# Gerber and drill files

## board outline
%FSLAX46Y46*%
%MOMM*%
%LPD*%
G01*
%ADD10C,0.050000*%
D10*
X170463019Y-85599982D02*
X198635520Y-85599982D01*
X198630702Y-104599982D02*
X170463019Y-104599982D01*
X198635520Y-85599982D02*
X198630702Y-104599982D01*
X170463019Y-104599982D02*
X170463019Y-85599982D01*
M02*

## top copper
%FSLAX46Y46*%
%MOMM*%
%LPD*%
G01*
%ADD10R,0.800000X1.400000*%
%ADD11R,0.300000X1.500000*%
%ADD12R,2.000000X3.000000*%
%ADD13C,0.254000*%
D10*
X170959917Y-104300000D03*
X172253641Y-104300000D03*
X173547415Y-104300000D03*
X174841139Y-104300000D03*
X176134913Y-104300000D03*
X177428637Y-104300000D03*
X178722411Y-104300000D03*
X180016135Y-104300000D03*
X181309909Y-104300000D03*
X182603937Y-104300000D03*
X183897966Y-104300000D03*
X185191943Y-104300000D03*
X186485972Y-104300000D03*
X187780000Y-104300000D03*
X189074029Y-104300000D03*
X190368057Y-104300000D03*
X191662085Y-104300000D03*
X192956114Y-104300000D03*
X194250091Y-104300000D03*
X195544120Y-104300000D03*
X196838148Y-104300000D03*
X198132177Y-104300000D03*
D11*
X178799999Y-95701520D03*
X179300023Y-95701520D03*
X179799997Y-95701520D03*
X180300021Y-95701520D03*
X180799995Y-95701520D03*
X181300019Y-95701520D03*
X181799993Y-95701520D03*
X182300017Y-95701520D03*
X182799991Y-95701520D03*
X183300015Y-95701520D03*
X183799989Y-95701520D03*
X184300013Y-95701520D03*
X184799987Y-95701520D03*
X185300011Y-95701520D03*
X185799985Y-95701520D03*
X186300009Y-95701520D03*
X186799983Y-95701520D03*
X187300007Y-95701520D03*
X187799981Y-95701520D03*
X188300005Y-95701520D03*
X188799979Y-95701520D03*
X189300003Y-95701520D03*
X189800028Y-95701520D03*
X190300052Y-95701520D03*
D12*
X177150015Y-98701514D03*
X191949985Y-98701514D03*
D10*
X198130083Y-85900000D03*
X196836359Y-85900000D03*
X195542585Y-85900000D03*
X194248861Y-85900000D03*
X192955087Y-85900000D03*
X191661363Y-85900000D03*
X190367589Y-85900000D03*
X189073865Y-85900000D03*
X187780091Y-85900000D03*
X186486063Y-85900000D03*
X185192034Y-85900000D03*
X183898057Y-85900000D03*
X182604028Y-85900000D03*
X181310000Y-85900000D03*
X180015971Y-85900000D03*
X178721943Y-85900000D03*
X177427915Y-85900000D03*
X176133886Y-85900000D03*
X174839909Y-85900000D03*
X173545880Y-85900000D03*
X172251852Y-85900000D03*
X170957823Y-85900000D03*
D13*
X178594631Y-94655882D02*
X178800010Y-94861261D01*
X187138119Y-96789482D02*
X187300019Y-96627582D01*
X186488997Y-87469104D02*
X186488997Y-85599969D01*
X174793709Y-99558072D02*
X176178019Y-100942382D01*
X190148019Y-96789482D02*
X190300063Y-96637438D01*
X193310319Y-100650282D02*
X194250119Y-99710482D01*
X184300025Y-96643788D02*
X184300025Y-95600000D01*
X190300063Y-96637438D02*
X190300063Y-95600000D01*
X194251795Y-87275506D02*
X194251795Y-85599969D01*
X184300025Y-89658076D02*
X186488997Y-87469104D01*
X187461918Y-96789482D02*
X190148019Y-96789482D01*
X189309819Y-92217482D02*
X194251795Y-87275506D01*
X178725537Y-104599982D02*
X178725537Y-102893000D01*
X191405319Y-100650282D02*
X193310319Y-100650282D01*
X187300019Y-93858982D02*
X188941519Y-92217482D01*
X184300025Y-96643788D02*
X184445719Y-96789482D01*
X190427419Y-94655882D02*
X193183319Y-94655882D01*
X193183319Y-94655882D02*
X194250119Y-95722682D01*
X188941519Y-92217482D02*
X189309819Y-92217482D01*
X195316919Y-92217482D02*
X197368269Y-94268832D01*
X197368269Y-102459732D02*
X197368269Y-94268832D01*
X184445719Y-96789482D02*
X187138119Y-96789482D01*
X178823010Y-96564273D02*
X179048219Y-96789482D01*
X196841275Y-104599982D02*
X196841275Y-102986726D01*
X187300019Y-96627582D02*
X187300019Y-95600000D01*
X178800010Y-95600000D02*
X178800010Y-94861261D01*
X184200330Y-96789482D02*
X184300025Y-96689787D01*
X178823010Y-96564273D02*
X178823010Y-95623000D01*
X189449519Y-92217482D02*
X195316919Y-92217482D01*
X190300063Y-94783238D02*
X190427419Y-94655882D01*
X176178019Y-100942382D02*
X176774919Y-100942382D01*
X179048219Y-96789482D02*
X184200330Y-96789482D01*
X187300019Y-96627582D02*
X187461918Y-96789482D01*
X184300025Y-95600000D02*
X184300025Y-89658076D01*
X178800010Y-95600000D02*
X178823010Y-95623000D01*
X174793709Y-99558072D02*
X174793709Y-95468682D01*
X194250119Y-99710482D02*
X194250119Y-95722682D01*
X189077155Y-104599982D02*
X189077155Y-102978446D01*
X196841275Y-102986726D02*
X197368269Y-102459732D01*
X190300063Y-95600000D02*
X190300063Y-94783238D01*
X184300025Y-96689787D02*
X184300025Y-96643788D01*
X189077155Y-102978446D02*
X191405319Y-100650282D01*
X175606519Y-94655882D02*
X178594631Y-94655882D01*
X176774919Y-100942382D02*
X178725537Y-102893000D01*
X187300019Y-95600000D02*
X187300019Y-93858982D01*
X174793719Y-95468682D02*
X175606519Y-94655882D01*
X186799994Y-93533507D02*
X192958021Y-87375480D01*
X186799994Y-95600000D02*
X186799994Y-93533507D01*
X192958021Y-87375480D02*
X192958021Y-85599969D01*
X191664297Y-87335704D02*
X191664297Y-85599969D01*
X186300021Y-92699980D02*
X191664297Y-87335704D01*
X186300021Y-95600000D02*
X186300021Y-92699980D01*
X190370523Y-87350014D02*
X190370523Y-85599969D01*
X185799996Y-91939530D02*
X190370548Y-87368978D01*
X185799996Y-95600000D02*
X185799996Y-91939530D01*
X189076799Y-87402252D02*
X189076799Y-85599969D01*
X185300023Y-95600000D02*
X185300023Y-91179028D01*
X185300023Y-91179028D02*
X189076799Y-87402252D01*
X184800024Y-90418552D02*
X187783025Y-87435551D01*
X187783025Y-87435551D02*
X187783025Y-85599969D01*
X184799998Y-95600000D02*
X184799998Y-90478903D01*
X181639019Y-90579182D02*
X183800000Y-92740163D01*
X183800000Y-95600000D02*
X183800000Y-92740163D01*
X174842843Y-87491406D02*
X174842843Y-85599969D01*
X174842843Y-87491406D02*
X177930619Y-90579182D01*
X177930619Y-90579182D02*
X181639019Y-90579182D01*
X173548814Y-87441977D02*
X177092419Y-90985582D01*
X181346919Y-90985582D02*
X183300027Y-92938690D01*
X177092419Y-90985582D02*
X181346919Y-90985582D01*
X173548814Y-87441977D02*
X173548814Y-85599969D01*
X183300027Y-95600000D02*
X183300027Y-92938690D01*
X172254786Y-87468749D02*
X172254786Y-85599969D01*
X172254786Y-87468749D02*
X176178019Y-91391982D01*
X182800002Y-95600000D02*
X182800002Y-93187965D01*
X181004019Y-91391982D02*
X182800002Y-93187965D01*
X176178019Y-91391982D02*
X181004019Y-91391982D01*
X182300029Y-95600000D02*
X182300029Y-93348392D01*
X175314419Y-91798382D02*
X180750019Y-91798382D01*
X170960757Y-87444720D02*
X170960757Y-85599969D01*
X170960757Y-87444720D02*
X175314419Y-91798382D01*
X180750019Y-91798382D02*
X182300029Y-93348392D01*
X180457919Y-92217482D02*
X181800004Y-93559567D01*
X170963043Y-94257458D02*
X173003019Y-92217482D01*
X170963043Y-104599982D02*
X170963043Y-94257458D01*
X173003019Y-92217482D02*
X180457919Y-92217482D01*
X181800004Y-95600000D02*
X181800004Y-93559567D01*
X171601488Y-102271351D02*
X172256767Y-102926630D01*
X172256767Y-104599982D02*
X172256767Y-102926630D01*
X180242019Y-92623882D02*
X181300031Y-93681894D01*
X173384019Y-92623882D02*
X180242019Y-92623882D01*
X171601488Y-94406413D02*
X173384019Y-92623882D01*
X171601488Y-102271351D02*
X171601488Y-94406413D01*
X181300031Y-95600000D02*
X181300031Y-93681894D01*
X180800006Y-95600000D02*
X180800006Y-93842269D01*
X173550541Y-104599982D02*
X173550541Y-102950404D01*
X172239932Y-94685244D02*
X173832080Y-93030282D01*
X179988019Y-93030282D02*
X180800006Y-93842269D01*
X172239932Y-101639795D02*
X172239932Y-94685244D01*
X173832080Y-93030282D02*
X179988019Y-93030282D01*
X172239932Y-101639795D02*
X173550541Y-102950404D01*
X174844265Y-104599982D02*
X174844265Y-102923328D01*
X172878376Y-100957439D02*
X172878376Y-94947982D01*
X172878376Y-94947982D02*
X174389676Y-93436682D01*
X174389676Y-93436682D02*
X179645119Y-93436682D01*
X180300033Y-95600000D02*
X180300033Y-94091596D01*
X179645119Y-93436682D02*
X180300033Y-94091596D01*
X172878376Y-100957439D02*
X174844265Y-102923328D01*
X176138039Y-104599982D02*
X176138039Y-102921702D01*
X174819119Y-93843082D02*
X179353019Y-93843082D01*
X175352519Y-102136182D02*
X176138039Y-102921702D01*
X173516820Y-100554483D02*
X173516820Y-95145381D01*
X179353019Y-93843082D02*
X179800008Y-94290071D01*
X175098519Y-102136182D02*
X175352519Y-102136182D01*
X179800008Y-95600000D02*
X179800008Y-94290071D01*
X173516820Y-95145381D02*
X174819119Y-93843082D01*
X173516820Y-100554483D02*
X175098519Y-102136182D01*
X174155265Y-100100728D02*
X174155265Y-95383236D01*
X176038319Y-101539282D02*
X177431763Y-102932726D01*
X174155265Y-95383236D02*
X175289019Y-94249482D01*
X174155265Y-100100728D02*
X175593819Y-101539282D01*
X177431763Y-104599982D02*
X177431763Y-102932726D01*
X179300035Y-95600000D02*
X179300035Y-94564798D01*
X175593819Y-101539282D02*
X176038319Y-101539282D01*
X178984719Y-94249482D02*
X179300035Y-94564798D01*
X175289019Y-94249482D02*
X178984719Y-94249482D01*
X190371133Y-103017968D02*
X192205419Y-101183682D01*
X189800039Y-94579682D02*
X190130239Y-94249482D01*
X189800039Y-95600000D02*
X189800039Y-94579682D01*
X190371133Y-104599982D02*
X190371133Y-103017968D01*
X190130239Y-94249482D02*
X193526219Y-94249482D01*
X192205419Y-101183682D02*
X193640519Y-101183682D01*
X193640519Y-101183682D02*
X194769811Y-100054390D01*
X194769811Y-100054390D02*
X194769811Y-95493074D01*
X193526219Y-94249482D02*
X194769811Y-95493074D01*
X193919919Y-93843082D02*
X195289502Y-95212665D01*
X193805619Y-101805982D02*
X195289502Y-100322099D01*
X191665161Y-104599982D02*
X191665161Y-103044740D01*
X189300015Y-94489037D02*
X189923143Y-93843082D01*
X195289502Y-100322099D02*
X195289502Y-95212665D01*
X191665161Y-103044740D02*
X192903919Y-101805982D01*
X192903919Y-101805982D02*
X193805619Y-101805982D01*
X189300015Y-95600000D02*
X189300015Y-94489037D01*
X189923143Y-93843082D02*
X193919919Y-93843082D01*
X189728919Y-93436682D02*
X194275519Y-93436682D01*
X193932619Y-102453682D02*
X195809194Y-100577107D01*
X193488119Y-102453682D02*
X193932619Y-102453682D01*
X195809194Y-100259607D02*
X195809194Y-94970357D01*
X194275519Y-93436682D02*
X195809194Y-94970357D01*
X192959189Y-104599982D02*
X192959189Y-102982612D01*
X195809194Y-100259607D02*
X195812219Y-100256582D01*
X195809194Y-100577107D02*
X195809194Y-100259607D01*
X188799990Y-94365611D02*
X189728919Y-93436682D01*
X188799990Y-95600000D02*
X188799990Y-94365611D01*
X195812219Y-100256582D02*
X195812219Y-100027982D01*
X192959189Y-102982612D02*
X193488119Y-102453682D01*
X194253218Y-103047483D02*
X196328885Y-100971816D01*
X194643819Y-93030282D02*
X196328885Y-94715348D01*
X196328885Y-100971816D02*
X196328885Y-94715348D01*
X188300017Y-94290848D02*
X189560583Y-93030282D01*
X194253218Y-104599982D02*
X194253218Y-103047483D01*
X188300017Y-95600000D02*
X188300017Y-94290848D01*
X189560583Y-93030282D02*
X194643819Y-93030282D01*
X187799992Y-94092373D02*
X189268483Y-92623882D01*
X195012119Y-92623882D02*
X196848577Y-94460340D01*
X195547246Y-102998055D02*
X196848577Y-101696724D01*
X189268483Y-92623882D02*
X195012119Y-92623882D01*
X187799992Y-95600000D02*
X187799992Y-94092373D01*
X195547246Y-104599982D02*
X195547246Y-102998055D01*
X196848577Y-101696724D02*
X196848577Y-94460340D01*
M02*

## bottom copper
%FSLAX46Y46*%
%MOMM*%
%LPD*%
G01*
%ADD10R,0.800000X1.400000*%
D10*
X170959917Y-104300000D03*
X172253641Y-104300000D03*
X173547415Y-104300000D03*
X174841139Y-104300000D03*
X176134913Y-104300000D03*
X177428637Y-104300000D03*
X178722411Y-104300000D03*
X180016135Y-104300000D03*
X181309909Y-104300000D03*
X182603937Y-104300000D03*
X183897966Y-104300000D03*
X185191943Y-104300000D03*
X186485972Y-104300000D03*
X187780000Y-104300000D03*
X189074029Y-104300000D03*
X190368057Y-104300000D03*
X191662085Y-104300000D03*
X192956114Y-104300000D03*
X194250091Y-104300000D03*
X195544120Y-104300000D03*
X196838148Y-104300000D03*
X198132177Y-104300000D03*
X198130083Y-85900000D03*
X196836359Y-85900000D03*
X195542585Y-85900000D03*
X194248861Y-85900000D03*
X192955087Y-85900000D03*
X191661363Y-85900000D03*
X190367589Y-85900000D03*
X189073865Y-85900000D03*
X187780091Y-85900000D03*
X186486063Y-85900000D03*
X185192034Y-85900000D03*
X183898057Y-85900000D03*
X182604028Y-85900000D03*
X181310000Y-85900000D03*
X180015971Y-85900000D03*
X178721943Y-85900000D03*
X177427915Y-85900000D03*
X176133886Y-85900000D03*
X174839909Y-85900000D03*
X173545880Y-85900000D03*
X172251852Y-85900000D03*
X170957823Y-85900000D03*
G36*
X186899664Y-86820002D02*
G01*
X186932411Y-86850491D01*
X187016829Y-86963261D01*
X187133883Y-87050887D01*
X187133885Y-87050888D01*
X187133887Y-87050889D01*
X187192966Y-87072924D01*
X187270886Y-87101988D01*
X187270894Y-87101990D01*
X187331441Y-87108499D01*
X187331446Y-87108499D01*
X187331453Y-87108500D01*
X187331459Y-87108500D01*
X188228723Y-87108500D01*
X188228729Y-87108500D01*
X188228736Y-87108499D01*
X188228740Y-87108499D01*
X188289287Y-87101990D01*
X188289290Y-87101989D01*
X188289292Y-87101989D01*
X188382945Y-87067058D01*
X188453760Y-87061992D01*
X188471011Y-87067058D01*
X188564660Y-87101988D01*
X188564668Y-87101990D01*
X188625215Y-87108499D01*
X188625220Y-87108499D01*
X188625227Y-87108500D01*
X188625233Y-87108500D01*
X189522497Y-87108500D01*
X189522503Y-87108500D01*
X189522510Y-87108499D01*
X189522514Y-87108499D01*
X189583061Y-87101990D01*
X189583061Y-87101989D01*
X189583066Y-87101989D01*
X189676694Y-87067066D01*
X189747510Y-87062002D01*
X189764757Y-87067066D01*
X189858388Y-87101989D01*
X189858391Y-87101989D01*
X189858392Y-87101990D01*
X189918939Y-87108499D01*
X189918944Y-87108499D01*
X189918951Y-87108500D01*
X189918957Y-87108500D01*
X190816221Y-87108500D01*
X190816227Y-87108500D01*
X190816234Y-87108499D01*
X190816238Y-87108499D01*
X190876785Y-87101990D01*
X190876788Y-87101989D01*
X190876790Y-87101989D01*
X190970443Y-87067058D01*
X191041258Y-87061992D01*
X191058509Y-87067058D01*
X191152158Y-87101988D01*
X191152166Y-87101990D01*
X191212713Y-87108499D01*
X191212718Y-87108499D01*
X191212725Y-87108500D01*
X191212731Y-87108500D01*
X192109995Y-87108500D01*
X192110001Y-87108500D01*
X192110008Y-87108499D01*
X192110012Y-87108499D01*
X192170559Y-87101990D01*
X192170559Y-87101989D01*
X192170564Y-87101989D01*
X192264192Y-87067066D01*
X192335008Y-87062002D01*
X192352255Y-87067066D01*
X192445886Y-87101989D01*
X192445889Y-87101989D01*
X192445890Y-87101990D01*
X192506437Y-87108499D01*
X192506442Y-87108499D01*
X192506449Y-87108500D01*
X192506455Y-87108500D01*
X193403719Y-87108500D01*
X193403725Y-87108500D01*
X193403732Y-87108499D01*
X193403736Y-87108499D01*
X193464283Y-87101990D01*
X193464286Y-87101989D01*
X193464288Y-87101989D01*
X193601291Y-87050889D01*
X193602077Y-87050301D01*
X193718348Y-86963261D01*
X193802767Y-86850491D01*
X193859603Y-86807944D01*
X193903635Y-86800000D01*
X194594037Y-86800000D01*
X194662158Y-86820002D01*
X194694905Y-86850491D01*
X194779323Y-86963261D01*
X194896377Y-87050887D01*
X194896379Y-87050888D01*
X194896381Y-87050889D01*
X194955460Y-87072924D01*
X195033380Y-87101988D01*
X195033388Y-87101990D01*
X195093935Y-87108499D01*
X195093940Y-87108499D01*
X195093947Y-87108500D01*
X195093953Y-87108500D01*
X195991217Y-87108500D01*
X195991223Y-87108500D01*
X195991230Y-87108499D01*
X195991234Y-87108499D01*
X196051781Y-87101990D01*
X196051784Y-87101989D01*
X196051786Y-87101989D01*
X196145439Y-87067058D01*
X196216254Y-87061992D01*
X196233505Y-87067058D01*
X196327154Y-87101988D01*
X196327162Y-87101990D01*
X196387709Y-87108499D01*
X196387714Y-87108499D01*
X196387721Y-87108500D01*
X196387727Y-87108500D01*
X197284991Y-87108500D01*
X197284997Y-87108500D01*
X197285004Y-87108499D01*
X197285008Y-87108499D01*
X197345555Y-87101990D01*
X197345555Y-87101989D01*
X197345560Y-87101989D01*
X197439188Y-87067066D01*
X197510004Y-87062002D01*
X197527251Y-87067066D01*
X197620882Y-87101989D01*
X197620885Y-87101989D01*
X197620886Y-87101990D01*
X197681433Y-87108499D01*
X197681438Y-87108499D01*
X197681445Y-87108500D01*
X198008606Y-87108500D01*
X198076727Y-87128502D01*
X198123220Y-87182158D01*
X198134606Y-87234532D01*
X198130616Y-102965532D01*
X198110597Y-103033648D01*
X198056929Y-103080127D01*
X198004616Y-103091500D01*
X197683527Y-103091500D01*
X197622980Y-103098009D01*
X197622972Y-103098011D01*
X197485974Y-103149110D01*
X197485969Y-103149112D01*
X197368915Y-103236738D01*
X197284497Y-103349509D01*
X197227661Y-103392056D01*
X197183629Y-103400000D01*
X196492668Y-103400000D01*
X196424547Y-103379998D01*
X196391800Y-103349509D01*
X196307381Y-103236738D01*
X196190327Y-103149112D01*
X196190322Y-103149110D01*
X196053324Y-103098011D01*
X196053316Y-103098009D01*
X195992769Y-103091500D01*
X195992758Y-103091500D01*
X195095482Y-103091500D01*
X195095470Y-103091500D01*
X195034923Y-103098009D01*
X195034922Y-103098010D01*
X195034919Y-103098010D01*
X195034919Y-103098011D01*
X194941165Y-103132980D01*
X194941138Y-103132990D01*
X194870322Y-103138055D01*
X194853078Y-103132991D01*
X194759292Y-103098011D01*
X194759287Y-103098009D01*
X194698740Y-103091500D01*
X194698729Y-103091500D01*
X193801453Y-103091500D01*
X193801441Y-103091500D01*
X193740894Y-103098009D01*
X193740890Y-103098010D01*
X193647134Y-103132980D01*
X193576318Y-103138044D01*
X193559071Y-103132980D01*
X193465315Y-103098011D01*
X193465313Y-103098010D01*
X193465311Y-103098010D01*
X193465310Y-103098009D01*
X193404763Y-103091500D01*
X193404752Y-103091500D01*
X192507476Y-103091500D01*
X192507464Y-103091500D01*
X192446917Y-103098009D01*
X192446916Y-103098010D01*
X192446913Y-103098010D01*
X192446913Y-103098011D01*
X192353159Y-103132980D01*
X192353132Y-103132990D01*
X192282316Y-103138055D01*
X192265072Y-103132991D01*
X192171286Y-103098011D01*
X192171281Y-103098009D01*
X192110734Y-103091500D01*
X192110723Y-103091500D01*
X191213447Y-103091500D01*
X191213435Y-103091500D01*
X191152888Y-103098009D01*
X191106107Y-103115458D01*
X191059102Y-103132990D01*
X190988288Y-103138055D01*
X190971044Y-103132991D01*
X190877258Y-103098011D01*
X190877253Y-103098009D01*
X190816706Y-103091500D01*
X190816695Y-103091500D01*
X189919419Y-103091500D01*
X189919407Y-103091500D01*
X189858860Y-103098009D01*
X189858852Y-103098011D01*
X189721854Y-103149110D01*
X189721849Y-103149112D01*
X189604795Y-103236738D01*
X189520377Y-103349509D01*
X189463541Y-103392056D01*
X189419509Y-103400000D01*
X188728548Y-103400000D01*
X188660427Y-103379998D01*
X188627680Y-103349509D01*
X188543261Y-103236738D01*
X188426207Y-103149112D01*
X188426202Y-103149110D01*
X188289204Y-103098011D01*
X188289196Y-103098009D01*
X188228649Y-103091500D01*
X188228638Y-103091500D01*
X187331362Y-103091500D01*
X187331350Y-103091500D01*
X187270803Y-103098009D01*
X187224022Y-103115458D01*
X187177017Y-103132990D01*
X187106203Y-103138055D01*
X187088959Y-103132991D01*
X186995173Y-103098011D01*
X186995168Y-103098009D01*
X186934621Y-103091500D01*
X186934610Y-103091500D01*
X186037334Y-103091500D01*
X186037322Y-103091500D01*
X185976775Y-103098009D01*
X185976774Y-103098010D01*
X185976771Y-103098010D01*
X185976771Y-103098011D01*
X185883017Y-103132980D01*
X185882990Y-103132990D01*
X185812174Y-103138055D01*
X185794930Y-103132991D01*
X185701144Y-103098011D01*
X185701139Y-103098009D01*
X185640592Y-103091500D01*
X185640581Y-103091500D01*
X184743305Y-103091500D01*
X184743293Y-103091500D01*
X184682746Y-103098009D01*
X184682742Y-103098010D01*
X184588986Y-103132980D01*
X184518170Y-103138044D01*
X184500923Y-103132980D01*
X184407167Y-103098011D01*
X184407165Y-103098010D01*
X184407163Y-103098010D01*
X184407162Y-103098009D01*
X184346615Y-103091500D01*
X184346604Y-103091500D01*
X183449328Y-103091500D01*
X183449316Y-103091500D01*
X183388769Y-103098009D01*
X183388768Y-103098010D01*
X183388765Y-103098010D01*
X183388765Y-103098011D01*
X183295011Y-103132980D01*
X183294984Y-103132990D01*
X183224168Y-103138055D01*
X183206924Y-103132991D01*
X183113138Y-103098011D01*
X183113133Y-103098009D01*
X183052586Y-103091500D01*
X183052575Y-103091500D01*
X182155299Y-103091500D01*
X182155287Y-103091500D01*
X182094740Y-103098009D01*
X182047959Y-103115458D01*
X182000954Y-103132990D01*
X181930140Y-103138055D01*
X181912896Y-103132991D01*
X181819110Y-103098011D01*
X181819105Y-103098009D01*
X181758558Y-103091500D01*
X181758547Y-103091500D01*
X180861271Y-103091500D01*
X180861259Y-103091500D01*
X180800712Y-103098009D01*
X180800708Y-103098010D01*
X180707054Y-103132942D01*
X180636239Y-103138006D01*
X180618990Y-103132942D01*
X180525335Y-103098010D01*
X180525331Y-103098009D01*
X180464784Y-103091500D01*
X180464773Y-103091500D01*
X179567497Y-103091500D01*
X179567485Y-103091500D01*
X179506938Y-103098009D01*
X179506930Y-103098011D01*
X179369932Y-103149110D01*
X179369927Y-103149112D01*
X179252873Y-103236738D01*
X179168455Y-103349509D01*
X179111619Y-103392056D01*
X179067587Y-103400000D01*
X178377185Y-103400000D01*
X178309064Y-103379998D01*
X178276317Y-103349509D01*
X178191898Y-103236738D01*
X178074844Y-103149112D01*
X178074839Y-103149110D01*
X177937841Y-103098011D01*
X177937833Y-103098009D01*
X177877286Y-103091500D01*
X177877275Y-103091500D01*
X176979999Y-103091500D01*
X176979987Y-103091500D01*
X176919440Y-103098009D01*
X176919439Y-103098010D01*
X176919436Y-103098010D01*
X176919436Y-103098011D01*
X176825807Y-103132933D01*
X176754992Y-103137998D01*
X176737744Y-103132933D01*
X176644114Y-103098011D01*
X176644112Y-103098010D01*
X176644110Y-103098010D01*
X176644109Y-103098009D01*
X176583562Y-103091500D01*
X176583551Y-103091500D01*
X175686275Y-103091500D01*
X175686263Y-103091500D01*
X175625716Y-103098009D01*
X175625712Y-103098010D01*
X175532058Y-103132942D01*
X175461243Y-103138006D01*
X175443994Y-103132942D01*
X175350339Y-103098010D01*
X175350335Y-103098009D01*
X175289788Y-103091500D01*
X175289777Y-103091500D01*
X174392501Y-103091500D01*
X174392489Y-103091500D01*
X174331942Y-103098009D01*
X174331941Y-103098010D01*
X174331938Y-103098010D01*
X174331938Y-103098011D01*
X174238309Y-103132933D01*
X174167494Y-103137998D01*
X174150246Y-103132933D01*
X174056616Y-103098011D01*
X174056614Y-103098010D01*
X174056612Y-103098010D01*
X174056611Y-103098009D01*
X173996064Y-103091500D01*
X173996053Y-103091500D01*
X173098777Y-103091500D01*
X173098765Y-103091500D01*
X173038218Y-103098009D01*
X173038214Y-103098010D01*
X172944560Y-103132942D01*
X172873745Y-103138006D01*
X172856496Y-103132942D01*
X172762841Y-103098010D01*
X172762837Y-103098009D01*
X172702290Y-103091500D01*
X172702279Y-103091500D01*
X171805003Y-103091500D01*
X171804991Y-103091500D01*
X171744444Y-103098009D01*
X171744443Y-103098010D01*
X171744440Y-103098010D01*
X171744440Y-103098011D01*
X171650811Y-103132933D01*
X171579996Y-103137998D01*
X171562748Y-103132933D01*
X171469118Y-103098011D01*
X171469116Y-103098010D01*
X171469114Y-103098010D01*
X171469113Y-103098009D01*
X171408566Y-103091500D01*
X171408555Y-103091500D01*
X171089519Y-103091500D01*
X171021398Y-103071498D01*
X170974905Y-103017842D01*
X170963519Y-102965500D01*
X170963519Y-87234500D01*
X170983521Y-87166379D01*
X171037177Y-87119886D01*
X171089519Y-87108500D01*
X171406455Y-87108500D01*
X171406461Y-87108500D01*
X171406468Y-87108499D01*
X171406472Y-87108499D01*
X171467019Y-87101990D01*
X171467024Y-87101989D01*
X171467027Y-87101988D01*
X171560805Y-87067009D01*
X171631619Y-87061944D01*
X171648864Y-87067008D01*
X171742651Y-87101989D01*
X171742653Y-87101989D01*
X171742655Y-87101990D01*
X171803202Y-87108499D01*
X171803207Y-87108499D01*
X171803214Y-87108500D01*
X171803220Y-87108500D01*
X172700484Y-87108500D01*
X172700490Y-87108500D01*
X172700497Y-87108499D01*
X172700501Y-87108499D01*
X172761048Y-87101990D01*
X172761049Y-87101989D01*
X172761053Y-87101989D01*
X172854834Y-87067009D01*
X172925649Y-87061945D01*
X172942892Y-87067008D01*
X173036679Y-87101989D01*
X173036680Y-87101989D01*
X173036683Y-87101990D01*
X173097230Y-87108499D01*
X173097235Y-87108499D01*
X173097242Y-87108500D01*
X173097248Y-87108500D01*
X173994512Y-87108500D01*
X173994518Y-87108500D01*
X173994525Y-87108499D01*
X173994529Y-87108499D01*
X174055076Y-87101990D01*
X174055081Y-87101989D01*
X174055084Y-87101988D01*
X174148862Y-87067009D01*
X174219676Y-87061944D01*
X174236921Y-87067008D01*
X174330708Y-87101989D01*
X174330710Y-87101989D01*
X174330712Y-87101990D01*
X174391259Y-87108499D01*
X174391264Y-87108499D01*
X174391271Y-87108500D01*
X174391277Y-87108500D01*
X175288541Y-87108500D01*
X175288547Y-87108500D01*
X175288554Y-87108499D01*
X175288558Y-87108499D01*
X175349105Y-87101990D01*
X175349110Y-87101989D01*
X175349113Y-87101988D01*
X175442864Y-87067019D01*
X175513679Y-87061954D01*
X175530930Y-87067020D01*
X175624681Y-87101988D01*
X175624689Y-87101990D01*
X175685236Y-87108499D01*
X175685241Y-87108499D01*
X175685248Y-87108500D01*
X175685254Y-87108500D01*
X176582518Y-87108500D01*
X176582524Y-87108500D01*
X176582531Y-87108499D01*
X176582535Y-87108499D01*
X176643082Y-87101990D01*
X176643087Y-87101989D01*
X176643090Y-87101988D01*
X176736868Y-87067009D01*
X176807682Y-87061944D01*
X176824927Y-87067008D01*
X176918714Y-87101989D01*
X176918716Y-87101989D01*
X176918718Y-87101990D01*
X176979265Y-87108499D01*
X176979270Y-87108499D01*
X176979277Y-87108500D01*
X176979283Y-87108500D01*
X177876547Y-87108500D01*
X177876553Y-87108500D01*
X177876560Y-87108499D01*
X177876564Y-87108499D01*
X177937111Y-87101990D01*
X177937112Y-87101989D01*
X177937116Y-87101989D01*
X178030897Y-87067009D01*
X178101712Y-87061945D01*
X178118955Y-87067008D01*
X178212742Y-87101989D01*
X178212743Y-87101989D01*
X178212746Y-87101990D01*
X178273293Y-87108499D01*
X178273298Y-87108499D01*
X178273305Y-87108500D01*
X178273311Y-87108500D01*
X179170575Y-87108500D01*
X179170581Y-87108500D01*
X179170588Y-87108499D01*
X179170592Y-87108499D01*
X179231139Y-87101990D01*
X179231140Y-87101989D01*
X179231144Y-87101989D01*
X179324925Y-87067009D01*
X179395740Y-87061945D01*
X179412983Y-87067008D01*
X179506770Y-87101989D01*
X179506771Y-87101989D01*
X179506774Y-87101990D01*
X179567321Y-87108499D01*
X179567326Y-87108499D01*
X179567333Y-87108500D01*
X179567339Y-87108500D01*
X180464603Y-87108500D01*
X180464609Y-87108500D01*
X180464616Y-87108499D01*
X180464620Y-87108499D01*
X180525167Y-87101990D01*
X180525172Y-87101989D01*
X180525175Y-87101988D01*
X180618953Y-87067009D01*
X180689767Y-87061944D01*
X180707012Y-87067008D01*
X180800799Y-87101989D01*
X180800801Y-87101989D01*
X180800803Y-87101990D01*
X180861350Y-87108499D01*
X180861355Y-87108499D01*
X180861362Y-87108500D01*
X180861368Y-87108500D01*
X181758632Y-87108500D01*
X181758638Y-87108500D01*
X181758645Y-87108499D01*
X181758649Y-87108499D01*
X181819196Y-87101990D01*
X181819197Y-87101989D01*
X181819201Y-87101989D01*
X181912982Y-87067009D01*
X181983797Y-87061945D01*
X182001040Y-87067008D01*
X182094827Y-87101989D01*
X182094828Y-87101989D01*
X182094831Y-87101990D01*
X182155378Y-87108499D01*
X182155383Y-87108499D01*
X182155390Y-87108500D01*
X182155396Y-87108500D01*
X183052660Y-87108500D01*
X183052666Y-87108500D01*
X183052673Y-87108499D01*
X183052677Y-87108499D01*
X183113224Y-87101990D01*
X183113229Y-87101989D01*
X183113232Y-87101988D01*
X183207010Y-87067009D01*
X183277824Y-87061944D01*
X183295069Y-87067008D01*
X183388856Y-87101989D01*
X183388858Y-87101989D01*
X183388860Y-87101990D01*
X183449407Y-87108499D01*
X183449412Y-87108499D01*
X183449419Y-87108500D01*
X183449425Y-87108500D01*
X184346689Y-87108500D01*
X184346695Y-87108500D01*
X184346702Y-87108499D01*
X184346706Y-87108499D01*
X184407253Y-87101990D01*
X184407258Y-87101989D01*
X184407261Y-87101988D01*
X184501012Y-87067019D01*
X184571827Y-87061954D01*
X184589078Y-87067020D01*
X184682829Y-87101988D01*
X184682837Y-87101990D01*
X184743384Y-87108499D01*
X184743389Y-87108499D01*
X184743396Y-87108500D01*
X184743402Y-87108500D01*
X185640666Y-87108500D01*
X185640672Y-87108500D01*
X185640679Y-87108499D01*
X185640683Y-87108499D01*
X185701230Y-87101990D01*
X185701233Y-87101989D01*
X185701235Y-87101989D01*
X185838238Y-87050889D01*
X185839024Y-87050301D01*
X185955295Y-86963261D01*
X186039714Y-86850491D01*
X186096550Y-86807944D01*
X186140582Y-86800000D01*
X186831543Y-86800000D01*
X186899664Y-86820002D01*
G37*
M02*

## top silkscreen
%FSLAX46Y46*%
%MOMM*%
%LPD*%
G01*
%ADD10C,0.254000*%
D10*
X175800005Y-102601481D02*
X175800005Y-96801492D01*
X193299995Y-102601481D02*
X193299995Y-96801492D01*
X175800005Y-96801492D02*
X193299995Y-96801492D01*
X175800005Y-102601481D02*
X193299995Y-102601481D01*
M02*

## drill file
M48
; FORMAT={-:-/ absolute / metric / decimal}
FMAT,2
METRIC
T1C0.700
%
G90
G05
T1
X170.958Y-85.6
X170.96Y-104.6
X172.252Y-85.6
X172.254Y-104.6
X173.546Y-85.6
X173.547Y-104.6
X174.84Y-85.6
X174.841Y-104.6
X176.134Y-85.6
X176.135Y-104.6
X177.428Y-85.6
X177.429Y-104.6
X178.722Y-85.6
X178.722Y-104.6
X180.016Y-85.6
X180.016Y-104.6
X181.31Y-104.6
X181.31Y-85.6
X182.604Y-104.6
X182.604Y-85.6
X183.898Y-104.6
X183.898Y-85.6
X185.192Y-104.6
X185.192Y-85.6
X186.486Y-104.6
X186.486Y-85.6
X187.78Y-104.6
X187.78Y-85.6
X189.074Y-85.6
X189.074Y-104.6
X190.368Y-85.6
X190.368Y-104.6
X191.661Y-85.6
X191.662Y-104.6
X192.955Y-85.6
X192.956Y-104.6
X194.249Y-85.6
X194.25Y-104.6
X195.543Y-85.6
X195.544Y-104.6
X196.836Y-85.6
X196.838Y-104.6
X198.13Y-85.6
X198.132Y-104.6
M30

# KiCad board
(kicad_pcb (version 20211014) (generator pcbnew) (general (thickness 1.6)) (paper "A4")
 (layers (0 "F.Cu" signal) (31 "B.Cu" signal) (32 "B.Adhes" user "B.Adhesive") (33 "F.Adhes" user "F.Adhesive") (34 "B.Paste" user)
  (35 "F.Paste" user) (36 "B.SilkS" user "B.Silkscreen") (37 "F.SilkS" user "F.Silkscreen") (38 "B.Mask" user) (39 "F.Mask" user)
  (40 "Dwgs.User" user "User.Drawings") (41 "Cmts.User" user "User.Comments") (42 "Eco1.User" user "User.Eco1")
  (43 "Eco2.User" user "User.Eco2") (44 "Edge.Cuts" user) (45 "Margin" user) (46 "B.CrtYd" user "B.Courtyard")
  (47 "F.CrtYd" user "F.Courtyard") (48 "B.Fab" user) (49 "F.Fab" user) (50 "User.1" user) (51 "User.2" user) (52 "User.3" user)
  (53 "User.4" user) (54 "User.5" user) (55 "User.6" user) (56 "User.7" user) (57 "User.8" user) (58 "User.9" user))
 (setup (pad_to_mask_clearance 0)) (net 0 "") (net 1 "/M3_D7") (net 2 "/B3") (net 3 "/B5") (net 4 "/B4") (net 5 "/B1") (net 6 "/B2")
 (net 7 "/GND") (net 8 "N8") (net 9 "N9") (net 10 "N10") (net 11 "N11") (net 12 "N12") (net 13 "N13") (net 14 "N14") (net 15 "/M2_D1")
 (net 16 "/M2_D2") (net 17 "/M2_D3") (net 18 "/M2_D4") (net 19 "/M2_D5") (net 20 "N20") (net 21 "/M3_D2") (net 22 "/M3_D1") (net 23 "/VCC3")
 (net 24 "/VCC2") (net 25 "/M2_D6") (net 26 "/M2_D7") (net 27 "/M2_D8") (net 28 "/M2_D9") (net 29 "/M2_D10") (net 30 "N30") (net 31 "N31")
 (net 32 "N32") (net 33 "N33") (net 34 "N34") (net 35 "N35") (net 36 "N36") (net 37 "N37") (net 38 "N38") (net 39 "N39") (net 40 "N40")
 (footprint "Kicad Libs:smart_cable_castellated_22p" (layer "F.Cu") (at 184.58 104.4 180)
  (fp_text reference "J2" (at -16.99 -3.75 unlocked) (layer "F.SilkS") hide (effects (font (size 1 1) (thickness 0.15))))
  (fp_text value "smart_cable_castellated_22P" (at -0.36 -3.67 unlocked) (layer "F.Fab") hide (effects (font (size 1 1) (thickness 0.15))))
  (pad "1" thru_hole rect (at 13.620083 -0.2 180) (size 0.8 1.4) (drill 0.7 (offset 0 0.3)) (layers *.Cu *.Mask) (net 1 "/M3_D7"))
  (pad "2" thru_hole rect (at 12.326359 -0.2 180) (size 0.8 1.4) (drill 0.7 (offset 0 0.3)) (layers *.Cu *.Mask) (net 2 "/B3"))
  (pad "3" thru_hole rect (at 11.032585 -0.2 180) (size 0.8 1.4) (drill 0.7 (offset 0 0.3)) (layers *.Cu *.Mask) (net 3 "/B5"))
  (pad "4" thru_hole rect (at 9.738861 -0.2 180) (size 0.8 1.4) (drill 0.7 (offset 0 0.3)) (layers *.Cu *.Mask) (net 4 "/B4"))
  (pad "5" thru_hole rect (at 8.445087 -0.2 180) (size 0.8 1.4) (drill 0.7 (offset 0 0.3)) (layers *.Cu *.Mask) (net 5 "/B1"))
  (pad "6" thru_hole rect (at 7.151363 -0.2 180) (size 0.8 1.4) (drill 0.7 (offset 0 0.3)) (layers *.Cu *.Mask) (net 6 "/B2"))
  (pad "7" thru_hole rect (at 5.857589 -0.2 180) (size 0.8 1.4) (drill 0.7 (offset 0 0.3)) (layers *.Cu *.Mask) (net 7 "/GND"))
  (pad "8" thru_hole rect (at 4.563865 -0.2 180) (size 0.8 1.4) (drill 0.7 (offset 0 0.3)) (layers *.Cu *.Mask) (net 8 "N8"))
  (pad "9" thru_hole rect (at 3.270091 -0.2 180) (size 0.8 1.4) (drill 0.7 (offset 0 0.3)) (layers *.Cu *.Mask) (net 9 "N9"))
  (pad "10" thru_hole rect (at 1.976063 -0.2 180) (size 0.8 1.4) (drill 0.7 (offset 0 0.3)) (layers *.Cu *.Mask) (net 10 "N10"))
  (pad "11" thru_hole rect (at 0.682034 -0.2 180) (size 0.8 1.4) (drill 0.7 (offset 0 0.3)) (layers *.Cu *.Mask) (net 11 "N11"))
  (pad "12" thru_hole rect (at -0.611943 -0.2 180) (size 0.8 1.4) (drill 0.7 (offset 0 0.3)) (layers *.Cu *.Mask) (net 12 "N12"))
  (pad "13" thru_hole rect (at -1.905972 -0.2 180) (size 0.8 1.4) (drill 0.7 (offset 0 0.3)) (layers *.Cu *.Mask) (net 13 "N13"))
  (pad "14" thru_hole rect (at -3.2 -0.2 180) (size 0.8 1.4) (drill 0.7 (offset 0 0.3)) (layers *.Cu *.Mask) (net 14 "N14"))
  (pad "15" thru_hole rect (at -4.494029 -0.2 180) (size 0.8 1.4) (drill 0.7 (offset 0 0.3)) (layers *.Cu *.Mask) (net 7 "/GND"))
  (pad "16" thru_hole rect (at -5.788057 -0.2 180) (size 0.8 1.4) (drill 0.7 (offset 0 0.3)) (layers *.Cu *.Mask) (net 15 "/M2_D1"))
  (pad "17" thru_hole rect (at -7.082085 -0.2 180) (size 0.8 1.4) (drill 0.7 (offset 0 0.3)) (layers *.Cu *.Mask) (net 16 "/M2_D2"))
  (pad "18" thru_hole rect (at -8.376114 -0.2 180) (size 0.8 1.4) (drill 0.7 (offset 0 0.3)) (layers *.Cu *.Mask) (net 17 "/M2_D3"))
  (pad "19" thru_hole rect (at -9.670091 -0.2 180) (size 0.8 1.4) (drill 0.7 (offset 0 0.3)) (layers *.Cu *.Mask) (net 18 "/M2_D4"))
  (pad "20" thru_hole rect (at -10.96412 -0.2 180) (size 0.8 1.4) (drill 0.7 (offset 0 0.3)) (layers *.Cu *.Mask) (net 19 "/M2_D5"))
  (pad "21" thru_hole rect (at -12.258148 -0.2 180) (size 0.8 1.4) (drill 0.7 (offset 0 0.3)) (layers *.Cu *.Mask) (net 7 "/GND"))
  (pad "22" thru_hole rect (at -13.552177 -0.2 180) (size 0.8 1.4) (drill 0.7 (offset 0 0.3)) (layers *.Cu *.Mask) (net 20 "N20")))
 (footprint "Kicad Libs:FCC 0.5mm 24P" (layer "F.Cu") (at 184.55 100.14)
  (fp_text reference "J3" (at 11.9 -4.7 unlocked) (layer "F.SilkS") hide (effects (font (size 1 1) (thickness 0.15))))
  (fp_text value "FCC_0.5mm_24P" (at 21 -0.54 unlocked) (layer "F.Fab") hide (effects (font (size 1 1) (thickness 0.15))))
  (fp_line (start -8.749995 2.461481) (end -8.749995 -3.338508) (layer "F.SilkS") (width 0.254))
  (fp_line (start 8.749995 2.461481) (end 8.749995 -3.338508) (layer "F.SilkS") (width 0.254))
  (fp_line (start -8.749995 -3.338508) (end 8.749995 -3.338508) (layer "F.SilkS") (width 0.254))
  (fp_line (start -8.749995 2.461481) (end 8.749995 2.461481) (layer "F.SilkS") (width 0.254))
  (pad "1" smd rect (at -5.750001 -4.43848) (size 0.3 1.5) (layers "F.Cu" "F.Paste" "F.Mask") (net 7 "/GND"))
  (pad "2" smd rect (at -5.249977 -4.43848) (size 0.3 1.5) (layers "F.Cu" "F.Paste" "F.Mask") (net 6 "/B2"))
  (pad "3" smd rect (at -4.750003 -4.43848) (size 0.3 1.5) (layers "F.Cu" "F.Paste" "F.Mask") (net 5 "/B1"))
  (pad "4" smd rect (at -4.249979 -4.43848) (size 0.3 1.5) (layers "F.Cu" "F.Paste" "F.Mask") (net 4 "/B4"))
  (pad "5" smd rect (at -3.750005 -4.43848) (size 0.3 1.5) (layers "F.Cu" "F.Paste" "F.Mask") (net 3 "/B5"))
  (pad "6" smd rect (at -3.249981 -4.43848) (size 0.3 1.5) (layers "F.Cu" "F.Paste" "F.Mask") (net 2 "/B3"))
  (pad "7" smd rect (at -2.750007 -4.43848) (size 0.3 1.5) (layers "F.Cu" "F.Paste" "F.Mask") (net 1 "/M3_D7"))
  (pad "8" smd rect (at -2.249983 -4.43848) (size 0.3 1.5) (layers "F.Cu" "F.Paste" "F.Mask") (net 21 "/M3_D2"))
  (pad "9" smd rect (at -1.750009 -4.43848) (size 0.3 1.5) (layers "F.Cu" "F.Paste" "F.Mask") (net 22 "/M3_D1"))
  (pad "10" smd rect (at -1.249985 -4.43848) (size 0.3 1.5) (layers "F.Cu" "F.Paste" "F.Mask") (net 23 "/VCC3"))
  (pad "11" smd rect (at -0.750011 -4.43848) (size 0.3 1.5) (layers "F.Cu" "F.Paste" "F.Mask") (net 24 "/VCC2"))
  (pad "12" smd rect (at -0.249987 -4.43848) (size 0.3 1.5) (layers "F.Cu" "F.Paste" "F.Mask") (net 7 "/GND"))
  (pad "13" smd rect (at 0.249987 -4.43848) (size 0.3 1.5) (layers "F.Cu" "F.Paste" "F.Mask") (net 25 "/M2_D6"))
  (pad "14" smd rect (at 0.750011 -4.43848) (size 0.3 1.5) (layers "F.Cu" "F.Paste" "F.Mask") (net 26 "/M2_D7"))
  (pad "15" smd rect (at 1.249985 -4.43848) (size 0.3 1.5) (layers "F.Cu" "F.Paste" "F.Mask") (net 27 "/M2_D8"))
  (pad "16" smd rect (at 1.750009 -4.43848) (size 0.3 1.5) (layers "F.Cu" "F.Paste" "F.Mask") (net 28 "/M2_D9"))
  (pad "17" smd rect (at 2.249983 -4.43848) (size 0.3 1.5) (layers "F.Cu" "F.Paste" "F.Mask") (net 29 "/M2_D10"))
  (pad "18" smd rect (at 2.750007 -4.43848) (size 0.3 1.5) (layers "F.Cu" "F.Paste" "F.Mask") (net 7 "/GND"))
  (pad "19" smd rect (at 3.249981 -4.43848) (size 0.3 1.5) (layers "F.Cu" "F.Paste" "F.Mask") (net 19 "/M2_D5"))
  (pad "20" smd rect (at 3.750005 -4.43848) (size 0.3 1.5) (layers "F.Cu" "F.Paste" "F.Mask") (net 18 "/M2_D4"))
  (pad "21" smd rect (at 4.249979 -4.43848) (size 0.3 1.5) (layers "F.Cu" "F.Paste" "F.Mask") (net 17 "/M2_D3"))
  (pad "22" smd rect (at 4.750003 -4.43848) (size 0.3 1.5) (layers "F.Cu" "F.Paste" "F.Mask") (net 16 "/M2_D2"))
  (pad "23" smd rect (at 5.250028 -4.43848) (size 0.3 1.5) (layers "F.Cu" "F.Paste" "F.Mask") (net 15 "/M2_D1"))
  (pad "24" smd rect (at 5.750052 -4.43848) (size 0.3 1.5) (layers "F.Cu" "F.Paste" "F.Mask") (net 7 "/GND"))
  (pad "A" smd rect (at -7.399985 -1.438486) (size 2 3) (layers "F.Cu" "F.Paste" "F.Mask"))
  (pad "A" smd rect (at 7.399985 -1.438486) (size 2 3) (layers "F.Cu" "F.Paste" "F.Mask")))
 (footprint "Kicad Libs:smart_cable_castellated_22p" (layer "F.Cu") (at 184.51 85.8)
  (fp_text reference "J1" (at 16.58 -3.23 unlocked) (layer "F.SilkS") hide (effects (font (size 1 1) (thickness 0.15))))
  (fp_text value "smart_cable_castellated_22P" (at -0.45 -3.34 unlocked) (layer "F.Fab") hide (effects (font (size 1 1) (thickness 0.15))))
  (pad "1" thru_hole rect (at 13.620083 -0.2) (size 0.8 1.4) (drill 0.7 (offset 0 0.3)) (layers *.Cu *.Mask) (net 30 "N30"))
  (pad "2" thru_hole rect (at 12.326359 -0.2) (size 0.8 1.4) (drill 0.7 (offset 0 0.3)) (layers *.Cu *.Mask) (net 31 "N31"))
  (pad "3" thru_hole rect (at 11.032585 -0.2) (size 0.8 1.4) (drill 0.7 (offset 0 0.3)) (layers *.Cu *.Mask) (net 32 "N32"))
  (pad "4" thru_hole rect (at 9.738861 -0.2) (size 0.8 1.4) (drill 0.7 (offset 0 0.3)) (layers *.Cu *.Mask) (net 7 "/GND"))
  (pad "5" thru_hole rect (at 8.445087 -0.2) (size 0.8 1.4) (drill 0.7 (offset 0 0.3)) (layers *.Cu *.Mask) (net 29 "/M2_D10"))
  (pad "6" thru_hole rect (at 7.151363 -0.2) (size 0.8 1.4) (drill 0.7 (offset 0 0.3)) (layers *.Cu *.Mask) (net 28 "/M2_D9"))
  (pad "7" thru_hole rect (at 5.857589 -0.2) (size 0.8 1.4) (drill 0.7 (offset 0 0.3)) (layers *.Cu *.Mask) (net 27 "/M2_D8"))
  (pad "8" thru_hole rect (at 4.563865 -0.2) (size 0.8 1.4) (drill 0.7 (offset 0 0.3)) (layers *.Cu *.Mask) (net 26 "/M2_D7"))
  (pad "9" thru_hole rect (at 3.270091 -0.2) (size 0.8 1.4) (drill 0.7 (offset 0 0.3)) (layers *.Cu *.Mask) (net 25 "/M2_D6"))
  (pad "10" thru_hole rect (at 1.976063 -0.2) (size 0.8 1.4) (drill 0.7 (offset 0 0.3)) (layers *.Cu *.Mask) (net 7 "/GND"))
  (pad "11" thru_hole rect (at 0.682034 -0.2) (size 0.8 1.4) (drill 0.7 (offset 0 0.3)) (layers *.Cu *.Mask) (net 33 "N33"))
  (pad "12" thru_hole rect (at -0.611943 -0.2) (size 0.8 1.4) (drill 0.7 (offset 0 0.3)) (layers *.Cu *.Mask) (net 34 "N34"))
  (pad "13" thru_hole rect (at -1.905972 -0.2) (size 0.8 1.4) (drill 0.7 (offset 0 0.3)) (layers *.Cu *.Mask) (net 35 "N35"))
  (pad "14" thru_hole rect (at -3.2 -0.2) (size 0.8 1.4) (drill 0.7 (offset 0 0.3)) (layers *.Cu *.Mask) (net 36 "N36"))
  (pad "15" thru_hole rect (at -4.494029 -0.2) (size 0.8 1.4) (drill 0.7 (offset 0 0.3)) (layers *.Cu *.Mask) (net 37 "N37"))
  (pad "16" thru_hole rect (at -5.788057 -0.2) (size 0.8 1.4) (drill 0.7 (offset 0 0.3)) (layers *.Cu *.Mask) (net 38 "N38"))
  (pad "17" thru_hole rect (at -7.082085 -0.2) (size 0.8 1.4) (drill 0.7 (offset 0 0.3)) (layers *.Cu *.Mask) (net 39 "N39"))
  (pad "18" thru_hole rect (at -8.376114 -0.2) (size 0.8 1.4) (drill 0.7 (offset 0 0.3)) (layers *.Cu *.Mask) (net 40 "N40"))
  (pad "19" thru_hole rect (at -9.670091 -0.2) (size 0.8 1.4) (drill 0.7 (offset 0 0.3)) (layers *.Cu *.Mask) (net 24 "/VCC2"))
  (pad "20" thru_hole rect (at -10.96412 -0.2) (size 0.8 1.4) (drill 0.7 (offset 0 0.3)) (layers *.Cu *.Mask) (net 23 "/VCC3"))
  (pad "21" thru_hole rect (at -12.258148 -0.2) (size 0.8 1.4) (drill 0.7 (offset 0 0.3)) (layers *.Cu *.Mask) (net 22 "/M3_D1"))
  (pad "22" thru_hole rect (at -13.552177 -0.2) (size 0.8 1.4) (drill 0.7 (offset 0 0.3)) (layers *.Cu *.Mask) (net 21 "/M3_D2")))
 (gr_line (start 170.463019 85.599982) (end 198.63552 85.599982) (layer "Edge.Cuts") (width 0.05))
 (gr_line (start 198.630702 104.599982) (end 170.463019 104.599982) (layer "Edge.Cuts") (width 0.05))
 (gr_line (start 198.63552 85.599982) (end 198.630702 104.599982) (layer "Edge.Cuts") (width 0.05))
 (gr_line (start 170.463019 104.599982) (end 170.463019 85.599982) (layer "Edge.Cuts") (width 0.05))
 (segment (start 178.594631 94.655882) (end 178.80001 94.861261) (width 0.254) (layer "F.Cu") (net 7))
 (segment (start 187.138119 96.789482) (end 187.300019 96.627582) (width 0.254) (layer "F.Cu") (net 7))
 (segment (start 186.488997 87.469104) (end 186.488997 85.599969) (width 0.254) (layer "F.Cu") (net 7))
 (segment (start 174.793709 99.558072) (end 176.178019 100.942382) (width 0.254) (layer "F.Cu") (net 7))
 (segment (start 190.148019 96.789482) (end 190.300063 96.637438) (width 0.254) (layer "F.Cu") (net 7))
 (segment (start 193.310319 100.650282) (end 194.250119 99.710482) (width 0.254) (layer "F.Cu") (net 7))
 (segment (start 184.300025 96.643788) (end 184.300025 95.6) (width 0.254) (layer "F.Cu") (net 7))
 (segment (start 190.300063 96.637438) (end 190.300063 95.6) (width 0.254) (layer "F.Cu") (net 7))
 (segment (start 194.251795 87.275506) (end 194.251795 85.599969) (width 0.254) (layer "F.Cu") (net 7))
 (segment (start 184.300025 89.658076) (end 186.488997 87.469104) (width 0.254) (layer "F.Cu") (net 7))
 (segment (start 187.461918 96.789482) (end 190.148019 96.789482) (width 0.254) (layer "F.Cu") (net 7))
 (segment (start 189.309819 92.217482) (end 194.251795 87.275506) (width 0.254) (layer "F.Cu") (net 7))
 (segment (start 178.725537 104.599982) (end 178.725537 102.893) (width 0.254) (layer "F.Cu") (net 7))
 (segment (start 191.405319 100.650282) (end 193.310319 100.650282) (width 0.254) (layer "F.Cu") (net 7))
 (segment (start 187.300019 93.858982) (end 188.941519 92.217482) (width 0.254) (layer "F.Cu") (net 7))
 (segment (start 184.300025 96.643788) (end 184.445719 96.789482) (width 0.254) (layer "F.Cu") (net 7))
 (segment (start 190.427419 94.655882) (end 193.183319 94.655882) (width 0.254) (layer "F.Cu") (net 7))
 (segment (start 193.183319 94.655882) (end 194.250119 95.722682) (width 0.254) (layer "F.Cu") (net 7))
 (segment (start 188.941519 92.217482) (end 189.309819 92.217482) (width 0.254) (layer "F.Cu") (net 7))
 (segment (start 195.316919 92.217482) (end 197.368269 94.268832) (width 0.254) (layer "F.Cu") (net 7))
 (segment (start 197.368269 102.459732) (end 197.368269 94.268832) (width 0.254) (layer "F.Cu") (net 7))
 (segment (start 184.445719 96.789482) (end 187.138119 96.789482) (width 0.254) (layer "F.Cu") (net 7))
 (segment (start 178.82301 96.564273) (end 179.048219 96.789482) (width 0.254) (layer "F.Cu") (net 7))
 (segment (start 196.841275 104.599982) (end 196.841275 102.986726) (width 0.254) (layer "F.Cu") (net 7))
 (segment (start 187.300019 96.627582) (end 187.300019 95.6) (width 0.254) (layer "F.Cu") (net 7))
 (segment (start 178.80001 95.6) (end 178.80001 94.861261) (width 0.254) (layer "F.Cu") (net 7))
 (segment (start 184.20033 96.789482) (end 184.300025 96.689787) (width 0.254) (layer "F.Cu") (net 7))
 (segment (start 178.82301 96.564273) (end 178.82301 95.623) (width 0.254) (layer "F.Cu") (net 7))
 (segment (start 189.449519 92.217482) (end 195.316919 92.217482) (width 0.254) (layer "F.Cu") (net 7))
 (segment (start 190.300063 94.783238) (end 190.427419 94.655882) (width 0.254) (layer "F.Cu") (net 7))
 (segment (start 176.178019 100.942382) (end 176.774919 100.942382) (width 0.254) (layer "F.Cu") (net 7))
 (segment (start 179.048219 96.789482) (end 184.20033 96.789482) (width 0.254) (layer "F.Cu") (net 7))
 (segment (start 187.300019 96.627582) (end 187.461918 96.789482) (width 0.254) (layer "F.Cu") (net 7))
 (segment (start 184.300025 95.6) (end 184.300025 89.658076) (width 0.254) (layer "F.Cu") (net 7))
 (segment (start 178.80001 95.6) (end 178.82301 95.623) (width 0.254) (layer "F.Cu") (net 7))
 (segment (start 174.793709 99.558072) (end 174.793709 95.468682) (width 0.254) (layer "F.Cu") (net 7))
 (segment (start 194.250119 99.710482) (end 194.250119 95.722682) (width 0.254) (layer "F.Cu") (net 7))
 (segment (start 189.077155 104.599982) (end 189.077155 102.978446) (width 0.254) (layer "F.Cu") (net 7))
 (segment (start 196.841275 102.986726) (end 197.368269 102.459732) (width 0.254) (layer "F.Cu") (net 7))
 (segment (start 190.300063 95.6) (end 190.300063 94.783238) (width 0.254) (layer "F.Cu") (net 7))
 (segment (start 184.300025 96.689787) (end 184.300025 96.643788) (width 0.254) (layer "F.Cu") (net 7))
 (segment (start 189.077155 102.978446) (end 191.405319 100.650282) (width 0.254) (layer "F.Cu") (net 7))
 (segment (start 175.606519 94.655882) (end 178.594631 94.655882) (width 0.254) (layer "F.Cu") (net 7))
 (segment (start 176.774919 100.942382) (end 178.725537 102.893) (width 0.254) (layer "F.Cu") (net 7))
 (segment (start 187.300019 95.6) (end 187.300019 93.858982) (width 0.254) (layer "F.Cu") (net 7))
 (segment (start 174.793719 95.468682) (end 175.606519 94.655882) (width 0.254) (layer "F.Cu") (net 7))
 (segment (start 186.799994 93.533507) (end 192.958021 87.37548) (width 0.254) (layer "F.Cu") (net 29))
 (segment (start 186.799994 95.6) (end 186.799994 93.533507) (width 0.254) (layer "F.Cu") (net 29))
 (segment (start 192.958021 87.37548) (end 192.958021 85.599969) (width 0.254) (layer "F.Cu") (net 29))
 (segment (start 191.664297 87.335704) (end 191.664297 85.599969) (width 0.254) (layer "F.Cu") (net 28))
 (segment (start 186.300021 92.69998) (end 191.664297 87.335704) (width 0.254) (layer "F.Cu") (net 28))
 (segment (start 186.300021 95.6) (end 186.300021 92.69998) (width 0.254) (layer "F.Cu") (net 28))
 (segment (start 190.370523 87.350014) (end 190.370523 85.599969) (width 0.254) (layer "F.Cu") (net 27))
 (segment (start 185.799996 91.93953) (end 190.370548 87.368978) (width 0.254) (layer "F.Cu") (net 27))
 (segment (start 185.799996 95.6) (end 185.799996 91.93953) (width 0.254) (layer "F.Cu") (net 27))
 (segment (start 189.076799 87.402252) (end 189.076799 85.599969) (width 0.254) (layer "F.Cu") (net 26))
 (segment (start 185.300023 95.6) (end 185.300023 91.179028) (width 0.254) (layer "F.Cu") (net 26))
 (segment (start 185.300023 91.179028) (end 189.076799 87.402252) (width 0.254) (layer "F.Cu") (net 26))
 (segment (start 184.800024 90.418552) (end 187.783025 87.435551) (width 0.254) (layer "F.Cu") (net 25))
 (segment (start 187.783025 87.435551) (end 187.783025 85.599969) (width 0.254) (layer "F.Cu") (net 25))
 (segment (start 184.799998 95.6) (end 184.799998 90.478903) (width 0.254) (layer "F.Cu") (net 25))
 (segment (start 181.639019 90.579182) (end 183.8 92.740163) (width 0.254) (layer "F.Cu") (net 24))
 (segment (start 183.8 95.6) (end 183.8 92.740163) (width 0.254) (layer "F.Cu") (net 24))
 (segment (start 174.842843 87.491406) (end 174.842843 85.599969) (width 0.254) (layer "F.Cu") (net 24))
 (segment (start 174.842843 87.491406) (end 177.930619 90.579182) (width 0.254) (layer "F.Cu") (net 24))
 (segment (start 177.930619 90.579182) (end 181.639019 90.579182) (width 0.254) (layer "F.Cu") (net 24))
 (segment (start 173.548814 87.441977) (end 177.092419 90.985582) (width 0.254) (layer "F.Cu") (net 23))
 (segment (start 181.346919 90.985582) (end 183.300027 92.93869) (width 0.254) (layer "F.Cu") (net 23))
 (segment (start 177.092419 90.985582) (end 181.346919 90.985582) (width 0.254) (layer "F.Cu") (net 23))
 (segment (start 173.548814 87.441977) (end 173.548814 85.599969) (width 0.254) (layer "F.Cu") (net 23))
 (segment (start 183.300027 95.6) (end 183.300027 92.93869) (width 0.254) (layer "F.Cu") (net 23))
 (segment (start 172.254786 87.468749) (end 172.254786 85.599969) (width 0.254) (layer "F.Cu") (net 22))
 (segment (start 172.254786 87.468749) (end 176.178019 91.391982) (width 0.254) (layer "F.Cu") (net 22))
 (segment (start 182.800002 95.6) (end 182.800002 93.187965) (width 0.254) (layer "F.Cu") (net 22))
 (segment (start 181.004019 91.391982) (end 182.800002 93.187965) (width 0.254) (layer "F.Cu") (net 22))
 (segment (start 176.178019 91.391982) (end 181.004019 91.391982) (width 0.254) (layer "F.Cu") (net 22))
 (segment (start 182.300029 95.6) (end 182.300029 93.348392) (width 0.254) (layer "F.Cu") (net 21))
 (segment (start 175.314419 91.798382) (end 180.750019 91.798382) (width 0.254) (layer "F.Cu") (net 21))
 (segment (start 170.960757 87.44472) (end 170.960757 85.599969) (width 0.254) (layer "F.Cu") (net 21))
 (segment (start 170.960757 87.44472) (end 175.314419 91.798382) (width 0.254) (layer "F.Cu") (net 21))
 (segment (start 180.750019 91.798382) (end 182.300029 93.348392) (width 0.254) (layer "F.Cu") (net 21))
 (segment (start 180.457919 92.217482) (end 181.800004 93.559567) (width 0.254) (layer "F.Cu") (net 1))
 (segment (start 170.963043 94.257458) (end 173.003019 92.217482) (width 0.254) (layer "F.Cu") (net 1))
 (segment (start 170.963043 104.599982) (end 170.963043 94.257458) (width 0.254) (layer "F.Cu") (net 1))
 (segment (start 173.003019 92.217482) (end 180.457919 92.217482) (width 0.254) (layer "F.Cu") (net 1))
 (segment (start 181.800004 95.6) (end 181.800004 93.559567) (width 0.254) (layer "F.Cu") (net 1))
 (segment (start 171.601488 102.271351) (end 172.256767 102.92663) (width 0.254) (layer "F.Cu") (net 2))
 (segment (start 172.256767 104.599982) (end 172.256767 102.92663) (width 0.254) (layer "F.Cu") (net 2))
 (segment (start 180.242019 92.623882) (end 181.300031 93.681894) (width 0.254) (layer "F.Cu") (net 2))
 (segment (start 173.384019 92.623882) (end 180.242019 92.623882) (width 0.254) (layer "F.Cu") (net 2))
 (segment (start 171.601488 94.406413) (end 173.384019 92.623882) (width 0.254) (layer "F.Cu") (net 2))
 (segment (start 171.601488 102.271351) (end 171.601488 94.406413) (width 0.254) (layer "F.Cu") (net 2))
 (segment (start 181.300031 95.6) (end 181.300031 93.681894) (width 0.254) (layer "F.Cu") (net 2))
 (segment (start 180.800006 95.6) (end 180.800006 93.842269) (width 0.254) (layer "F.Cu") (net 3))
 (segment (start 173.550541 104.599982) (end 173.550541 102.950404) (width 0.254) (layer "F.Cu") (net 3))
 (segment (start 172.239932 94.685244) (end 173.83208 93.030282) (width 0.254) (layer "F.Cu") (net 3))
 (segment (start 179.988019 93.030282) (end 180.800006 93.842269) (width 0.254) (layer "F.Cu") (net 3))
 (segment (start 172.239932 101.639795) (end 172.239932 94.685244) (width 0.254) (layer "F.Cu") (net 3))
 (segment (start 173.83208 93.030282) (end 179.988019 93.030282) (width 0.254) (layer "F.Cu") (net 3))
 (segment (start 172.239932 101.639795) (end 173.550541 102.950404) (width 0.254) (layer "F.Cu") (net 3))
 (segment (start 174.844265 104.599982) (end 174.844265 102.923328) (width 0.254) (layer "F.Cu") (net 4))
 (segment (start 172.878376 100.957439) (end 172.878376 94.947982) (width 0.254) (layer "F.Cu") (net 4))
 (segment (start 172.878376 94.947982) (end 174.389676 93.436682) (width 0.254) (layer "F.Cu") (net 4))
 (segment (start 174.389676 93.436682) (end 179.645119 93.436682) (width 0.254) (layer "F.Cu") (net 4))
 (segment (start 180.300033 95.6) (end 180.300033 94.091596) (width 0.254) (layer "F.Cu") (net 4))
 (segment (start 179.645119 93.436682) (end 180.300033 94.091596) (width 0.254) (layer "F.Cu") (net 4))
 (segment (start 172.878376 100.957439) (end 174.844265 102.923328) (width 0.254) (layer "F.Cu") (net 4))
 (segment (start 176.138039 104.599982) (end 176.138039 102.921702) (width 0.254) (layer "F.Cu") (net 5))
 (segment (start 174.819119 93.843082) (end 179.353019 93.843082) (width 0.254) (layer "F.Cu") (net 5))
 (segment (start 175.352519 102.136182) (end 176.138039 102.921702) (width 0.254) (layer "F.Cu") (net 5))
 (segment (start 173.51682 100.554483) (end 173.51682 95.145381) (width 0.254) (layer "F.Cu") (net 5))
 (segment (start 179.353019 93.843082) (end 179.800008 94.290071) (width 0.254) (layer "F.Cu") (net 5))
 (segment (start 175.098519 102.136182) (end 175.352519 102.136182) (width 0.254) (layer "F.Cu") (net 5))
 (segment (start 179.800008 95.6) (end 179.800008 94.290071) (width 0.254) (layer "F.Cu") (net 5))
 (segment (start 173.51682 95.145381) (end 174.819119 93.843082) (width 0.254) (layer "F.Cu") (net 5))
 (segment (start 173.51682 100.554483) (end 175.098519 102.136182) (width 0.254) (layer "F.Cu") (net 5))
 (segment (start 174.155265 100.100728) (end 174.155265 95.383236) (width 0.254) (layer "F.Cu") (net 6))
 (segment (start 176.038319 101.539282) (end 177.431763 102.932726) (width 0.254) (layer "F.Cu") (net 6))
 (segment (start 174.155265 95.383236) (end 175.289019 94.249482) (width 0.254) (layer "F.Cu") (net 6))
 (segment (start 174.155265 100.100728) (end 175.593819 101.539282) (width 0.254) (layer "F.Cu") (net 6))
 (segment (start 177.431763 104.599982) (end 177.431763 102.932726) (width 0.254) (layer "F.Cu") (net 6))
 (segment (start 179.300035 95.6) (end 179.300035 94.564798) (width 0.254) (layer "F.Cu") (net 6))
 (segment (start 175.593819 101.539282) (end 176.038319 101.539282) (width 0.254) (layer "F.Cu") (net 6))
 (segment (start 178.984719 94.249482) (end 179.300035 94.564798) (width 0.254) (layer "F.Cu") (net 6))
 (segment (start 175.289019 94.249482) (end 178.984719 94.249482) (width 0.254) (layer "F.Cu") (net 6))
 (segment (start 190.371133 103.017968) (end 192.205419 101.183682) (width 0.254) (layer "F.Cu") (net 15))
 (segment (start 189.800039 94.579682) (end 190.130239 94.249482) (width 0.254) (layer "F.Cu") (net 15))
 (segment (start 189.800039 95.6) (end 189.800039 94.579682) (width 0.254) (layer "F.Cu") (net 15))
 (segment (start 190.371133 104.599982) (end 190.371133 103.017968) (width 0.254) (layer "F.Cu") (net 15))
 (segment (start 190.130239 94.249482) (end 193.526219 94.249482) (width 0.254) (layer "F.Cu") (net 15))
 (segment (start 192.205419 101.183682) (end 193.640519 101.183682) (width 0.254) (layer "F.Cu") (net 15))
 (segment (start 193.640519 101.183682) (end 194.769811 100.05439) (width 0.254) (layer "F.Cu") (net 15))
 (segment (start 194.769811 100.05439) (end 194.769811 95.493074) (width 0.254) (layer "F.Cu") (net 15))
 (segment (start 193.526219 94.249482) (end 194.769811 95.493074) (width 0.254) (layer "F.Cu") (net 15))
 (segment (start 193.919919 93.843082) (end 195.289502 95.212665) (width 0.254) (layer "F.Cu") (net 16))
 (segment (start 193.805619 101.805982) (end 195.289502 100.322099) (width 0.254) (layer "F.Cu") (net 16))
 (segment (start 191.665161 104.599982) (end 191.665161 103.04474) (width 0.254) (layer "F.Cu") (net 16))
 (segment (start 189.300015 94.489037) (end 189.923143 93.843082) (width 0.254) (layer "F.Cu") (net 16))
 (segment (start 195.289502 100.322099) (end 195.289502 95.212665) (width 0.254) (layer "F.Cu") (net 16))
 (segment (start 191.665161 103.04474) (end 192.903919 101.805982) (width 0.254) (layer "F.Cu") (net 16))
 (segment (start 192.903919 101.805982) (end 193.805619 101.805982) (width 0.254) (layer "F.Cu") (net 16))
 (segment (start 189.300015 95.6) (end 189.300015 94.489037) (width 0.254) (layer "F.Cu") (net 16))
 (segment (start 189.923143 93.843082) (end 193.919919 93.843082) (width 0.254) (layer "F.Cu") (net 16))
 (segment (start 189.728919 93.436682) (end 194.275519 93.436682) (width 0.254) (layer "F.Cu") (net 17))
 (segment (start 193.932619 102.453682) (end 195.809194 100.577107) (width 0.254) (layer "F.Cu") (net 17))
 (segment (start 193.488119 102.453682) (end 193.932619 102.453682) (width 0.254) (layer "F.Cu") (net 17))
 (segment (start 195.809194 100.259607) (end 195.809194 94.970357) (width 0.254) (layer "F.Cu") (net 17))
 (segment (start 194.275519 93.436682) (end 195.809194 94.970357) (width 0.254) (layer "F.Cu") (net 17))
 (segment (start 192.959189 104.599982) (end 192.959189 102.982612) (width 0.254) (layer "F.Cu") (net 17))
 (segment (start 195.809194 100.259607) (end 195.812219 100.256582) (width 0.254) (layer "F.Cu") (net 17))
 (segment (start 195.809194 100.577107) (end 195.809194 100.259607) (width 0.254) (layer "F.Cu") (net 17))
 (segment (start 188.79999 94.365611) (end 189.728919 93.436682) (width 0.254) (layer "F.Cu") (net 17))
 (segment (start 188.79999 95.6) (end 188.79999 94.365611) (width 0.254) (layer "F.Cu") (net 17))
 (segment (start 195.812219 100.256582) (end 195.812219 100.027982) (width 0.254) (layer "F.Cu") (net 17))
 (segment (start 192.959189 102.982612) (end 193.488119 102.453682) (width 0.254) (layer "F.Cu") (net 17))
 (segment (start 194.253218 103.047483) (end 196.328885 100.971816) (width 0.254) (layer "F.Cu") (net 18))
 (segment (start 194.643819 93.030282) (end 196.328885 94.715348) (width 0.254) (layer "F.Cu") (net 18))
 (segment (start 196.328885 100.971816) (end 196.328885 94.715348) (width 0.254) (layer "F.Cu") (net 18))
 (segment (start 188.300017 94.290848) (end 189.560583 93.030282) (width 0.254) (layer "F.Cu") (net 18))
 (segment (start 194.253218 104.599982) (end 194.253218 103.047483) (width 0.254) (layer "F.Cu") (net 18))
 (segment (start 188.300017 95.6) (end 188.300017 94.290848) (width 0.254) (layer "F.Cu") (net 18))
 (segment (start 189.560583 93.030282) (end 194.643819 93.030282) (width 0.254) (layer "F.Cu") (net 18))
 (segment (start 187.799992 94.092373) (end 189.268483 92.623882) (width 0.254) (layer "F.Cu") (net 19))
 (segment (start 195.012119 92.623882) (end 196.848577 94.46034) (width 0.254) (layer "F.Cu") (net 19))
 (segment (start 195.547246 102.998055) (end 196.848577 101.696724) (width 0.254) (layer "F.Cu") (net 19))
 (segment (start 189.268483 92.623882) (end 195.012119 92.623882) (width 0.254) (layer "F.Cu") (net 19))
 (segment (start 187.799992 95.6) (end 187.799992 94.092373) (width 0.254) (layer "F.Cu") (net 19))
 (segment (start 195.547246 104.599982) (end 195.547246 102.998055) (width 0.254) (layer "F.Cu") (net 19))
 (segment (start 196.848577 101.696724) (end 196.848577 94.46034) (width 0.254) (layer "F.Cu") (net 19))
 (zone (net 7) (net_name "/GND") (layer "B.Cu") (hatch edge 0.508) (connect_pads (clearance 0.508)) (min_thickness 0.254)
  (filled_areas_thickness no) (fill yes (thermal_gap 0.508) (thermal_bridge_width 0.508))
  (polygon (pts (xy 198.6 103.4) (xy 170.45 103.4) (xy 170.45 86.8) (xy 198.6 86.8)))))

